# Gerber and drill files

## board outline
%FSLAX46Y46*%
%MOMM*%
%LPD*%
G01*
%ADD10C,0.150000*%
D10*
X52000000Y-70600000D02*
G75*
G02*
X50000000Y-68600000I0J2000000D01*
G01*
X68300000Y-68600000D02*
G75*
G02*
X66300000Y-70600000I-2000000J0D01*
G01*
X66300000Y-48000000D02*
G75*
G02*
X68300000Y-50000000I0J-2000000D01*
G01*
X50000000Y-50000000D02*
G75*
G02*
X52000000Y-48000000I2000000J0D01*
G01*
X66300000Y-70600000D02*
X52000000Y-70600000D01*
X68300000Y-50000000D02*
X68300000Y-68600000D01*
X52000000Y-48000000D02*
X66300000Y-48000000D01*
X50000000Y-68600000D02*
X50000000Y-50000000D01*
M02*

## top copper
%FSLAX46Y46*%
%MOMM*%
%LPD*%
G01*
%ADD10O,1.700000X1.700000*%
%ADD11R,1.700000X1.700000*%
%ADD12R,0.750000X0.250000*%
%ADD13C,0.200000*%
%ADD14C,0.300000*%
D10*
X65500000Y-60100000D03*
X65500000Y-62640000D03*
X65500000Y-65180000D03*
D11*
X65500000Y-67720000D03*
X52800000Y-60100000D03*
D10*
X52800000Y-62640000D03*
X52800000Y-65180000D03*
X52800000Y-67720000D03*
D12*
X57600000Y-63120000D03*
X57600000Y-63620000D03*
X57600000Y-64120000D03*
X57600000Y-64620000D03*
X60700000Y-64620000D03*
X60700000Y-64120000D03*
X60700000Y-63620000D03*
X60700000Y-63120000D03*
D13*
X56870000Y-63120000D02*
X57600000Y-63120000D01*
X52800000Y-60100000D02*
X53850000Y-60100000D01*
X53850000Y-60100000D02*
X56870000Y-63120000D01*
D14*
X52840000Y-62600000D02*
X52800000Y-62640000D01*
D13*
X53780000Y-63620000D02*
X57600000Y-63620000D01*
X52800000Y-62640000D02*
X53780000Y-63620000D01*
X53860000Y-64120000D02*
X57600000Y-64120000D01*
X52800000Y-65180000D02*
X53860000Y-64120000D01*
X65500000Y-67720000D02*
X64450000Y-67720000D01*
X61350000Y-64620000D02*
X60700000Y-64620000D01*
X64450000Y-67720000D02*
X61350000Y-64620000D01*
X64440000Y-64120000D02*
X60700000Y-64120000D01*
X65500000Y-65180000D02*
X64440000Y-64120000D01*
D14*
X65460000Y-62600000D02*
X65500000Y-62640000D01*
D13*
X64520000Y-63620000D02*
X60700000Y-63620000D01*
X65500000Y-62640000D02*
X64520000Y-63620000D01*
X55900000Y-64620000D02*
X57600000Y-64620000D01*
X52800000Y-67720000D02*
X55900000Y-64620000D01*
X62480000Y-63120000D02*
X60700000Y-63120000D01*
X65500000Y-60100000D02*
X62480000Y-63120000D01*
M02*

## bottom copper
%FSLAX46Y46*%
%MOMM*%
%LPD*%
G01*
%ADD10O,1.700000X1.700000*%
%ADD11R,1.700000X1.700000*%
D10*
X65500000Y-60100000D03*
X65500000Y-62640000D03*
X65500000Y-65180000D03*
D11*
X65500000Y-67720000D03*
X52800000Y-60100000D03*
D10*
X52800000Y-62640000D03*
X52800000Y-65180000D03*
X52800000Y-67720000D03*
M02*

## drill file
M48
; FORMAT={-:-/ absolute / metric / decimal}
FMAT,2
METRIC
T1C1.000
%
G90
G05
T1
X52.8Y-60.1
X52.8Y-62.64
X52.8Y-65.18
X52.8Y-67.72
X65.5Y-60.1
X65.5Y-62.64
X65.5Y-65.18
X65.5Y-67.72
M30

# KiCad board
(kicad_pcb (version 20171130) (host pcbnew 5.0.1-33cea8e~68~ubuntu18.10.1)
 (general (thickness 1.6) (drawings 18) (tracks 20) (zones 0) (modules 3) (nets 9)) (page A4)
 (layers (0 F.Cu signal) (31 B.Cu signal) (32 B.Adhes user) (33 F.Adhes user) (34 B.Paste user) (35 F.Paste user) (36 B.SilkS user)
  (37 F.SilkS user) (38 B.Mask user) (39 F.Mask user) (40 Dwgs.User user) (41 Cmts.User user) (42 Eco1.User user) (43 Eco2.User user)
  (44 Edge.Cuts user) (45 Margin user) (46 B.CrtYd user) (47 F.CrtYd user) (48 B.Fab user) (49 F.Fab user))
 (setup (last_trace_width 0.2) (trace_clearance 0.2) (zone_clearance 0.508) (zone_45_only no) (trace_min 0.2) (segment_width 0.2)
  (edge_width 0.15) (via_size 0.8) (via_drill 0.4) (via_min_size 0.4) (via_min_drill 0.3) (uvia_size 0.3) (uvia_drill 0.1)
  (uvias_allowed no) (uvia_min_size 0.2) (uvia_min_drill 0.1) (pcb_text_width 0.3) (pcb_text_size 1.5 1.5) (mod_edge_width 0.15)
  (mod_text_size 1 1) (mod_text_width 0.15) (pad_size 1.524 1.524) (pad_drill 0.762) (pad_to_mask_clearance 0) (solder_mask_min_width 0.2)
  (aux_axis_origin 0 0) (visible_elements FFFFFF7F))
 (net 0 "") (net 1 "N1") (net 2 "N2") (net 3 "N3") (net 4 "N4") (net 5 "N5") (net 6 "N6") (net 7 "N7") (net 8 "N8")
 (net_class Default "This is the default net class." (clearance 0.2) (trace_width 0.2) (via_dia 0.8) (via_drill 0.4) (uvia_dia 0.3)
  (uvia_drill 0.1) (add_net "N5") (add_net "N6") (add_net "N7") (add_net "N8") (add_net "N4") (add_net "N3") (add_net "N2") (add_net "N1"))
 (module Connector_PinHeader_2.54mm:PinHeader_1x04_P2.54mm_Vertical (layer F.Cu) (at 65.5 67.72 180)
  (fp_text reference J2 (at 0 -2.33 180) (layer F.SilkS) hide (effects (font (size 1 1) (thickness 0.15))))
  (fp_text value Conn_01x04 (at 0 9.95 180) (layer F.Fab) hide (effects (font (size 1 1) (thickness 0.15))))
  (pad 4 thru_hole oval (at 0 7.62 180) (size 1.7 1.7) (drill 1) (layers *.Cu *.Mask) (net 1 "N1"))
  (pad 3 thru_hole oval (at 0 5.08 180) (size 1.7 1.7) (drill 1) (layers *.Cu *.Mask) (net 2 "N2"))
  (pad 2 thru_hole oval (at 0 2.54 180) (size 1.7 1.7) (drill 1) (layers *.Cu *.Mask) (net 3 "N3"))
  (pad 1 thru_hole rect (at 0 0 180) (size 1.7 1.7) (drill 1) (layers *.Cu *.Mask) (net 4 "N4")))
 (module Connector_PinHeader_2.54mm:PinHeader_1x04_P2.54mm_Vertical (layer F.Cu) (at 52.8 60.1)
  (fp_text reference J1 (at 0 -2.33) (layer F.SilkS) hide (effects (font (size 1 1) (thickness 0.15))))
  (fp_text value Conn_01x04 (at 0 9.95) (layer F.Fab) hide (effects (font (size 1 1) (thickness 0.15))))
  (pad 1 thru_hole rect (at 0 0) (size 1.7 1.7) (drill 1) (layers *.Cu *.Mask) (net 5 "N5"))
  (pad 2 thru_hole oval (at 0 2.54) (size 1.7 1.7) (drill 1) (layers *.Cu *.Mask) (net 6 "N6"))
  (pad 3 thru_hole oval (at 0 5.08) (size 1.7 1.7) (drill 1) (layers *.Cu *.Mask) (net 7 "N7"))
  (pad 4 thru_hole oval (at 0 7.62) (size 1.7 1.7) (drill 1) (layers *.Cu *.Mask) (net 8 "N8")))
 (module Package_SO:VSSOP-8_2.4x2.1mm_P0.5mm (layer F.Cu) (at 59.15 63.87)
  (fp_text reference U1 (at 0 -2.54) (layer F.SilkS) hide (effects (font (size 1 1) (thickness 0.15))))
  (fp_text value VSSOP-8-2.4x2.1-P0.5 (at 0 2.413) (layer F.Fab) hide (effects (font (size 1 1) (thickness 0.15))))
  (pad 1 smd rect (at -1.55 -0.75) (size 0.75 0.25) (layers F.Cu F.Paste F.Mask) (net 5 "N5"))
  (pad 2 smd rect (at -1.55 -0.25) (size 0.75 0.25) (layers F.Cu F.Paste F.Mask) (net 6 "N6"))
  (pad 3 smd rect (at -1.55 0.25) (size 0.75 0.25) (layers F.Cu F.Paste F.Mask) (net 7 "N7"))
  (pad 4 smd rect (at -1.55 0.75) (size 0.75 0.25) (layers F.Cu F.Paste F.Mask) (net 8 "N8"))
  (pad 5 smd rect (at 1.55 0.75) (size 0.75 0.25) (layers F.Cu F.Paste F.Mask) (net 4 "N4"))
  (pad 6 smd rect (at 1.55 0.25) (size 0.75 0.25) (layers F.Cu F.Paste F.Mask) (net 3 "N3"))
  (pad 7 smd rect (at 1.55 -0.25) (size 0.75 0.25) (layers F.Cu F.Paste F.Mask) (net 2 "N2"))
  (pad 8 smd rect (at 1.55 -0.75) (size 0.75 0.25) (layers F.Cu F.Paste F.Mask) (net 1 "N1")))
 (gr_arc (start 52 68.6) (end 50 68.6) (angle -90) (layer Edge.Cuts) (width 0.15))
 (gr_arc (start 66.3 68.6) (end 66.3 70.6) (angle -90) (layer Edge.Cuts) (width 0.15))
 (gr_arc (start 66.3 50) (end 68.3 50) (angle -90) (layer Edge.Cuts) (width 0.15))
 (gr_arc (start 52 50) (end 52 48) (angle -90) (layer Edge.Cuts) (width 0.15))
 (gr_line (start 66.3 70.6) (end 52 70.6) (layer Edge.Cuts) (width 0.15))
 (gr_line (start 68.3 50) (end 68.3 68.6) (layer Edge.Cuts) (width 0.15))
 (gr_line (start 52 48) (end 66.3 48) (layer Edge.Cuts) (width 0.15))
 (gr_line (start 50 68.6) (end 50 50) (layer Edge.Cuts) (width 0.15))
 (segment (start 56.87 63.12) (end 57.6 63.12) (width 0.2) (layer F.Cu) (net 5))
 (segment (start 52.8 60.1) (end 53.85 60.1) (width 0.2) (layer F.Cu) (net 5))
 (segment (start 53.85 60.1) (end 56.87 63.12) (width 0.2) (layer F.Cu) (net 5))
 (segment (start 52.84 62.6) (end 52.8 62.64) (width 0.3) (layer F.Cu) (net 6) (status 30))
 (segment (start 53.78 63.62) (end 57.6 63.62) (width 0.2) (layer F.Cu) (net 6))
 (segment (start 52.8 62.64) (end 53.78 63.62) (width 0.2) (layer F.Cu) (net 6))
 (segment (start 53.86 64.12) (end 57.6 64.12) (width 0.2) (layer F.Cu) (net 7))
 (segment (start 52.8 65.18) (end 53.86 64.12) (width 0.2) (layer F.Cu) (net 7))
 (segment (start 65.5 67.72) (end 64.45 67.72) (width 0.2) (layer F.Cu) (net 4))
 (segment (start 61.35 64.62) (end 60.7 64.62) (width 0.2) (layer F.Cu) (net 4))
 (segment (start 64.45 67.72) (end 61.35 64.62) (width 0.2) (layer F.Cu) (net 4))
 (segment (start 64.44 64.12) (end 60.7 64.12) (width 0.2) (layer F.Cu) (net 3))
 (segment (start 65.5 65.18) (end 64.44 64.12) (width 0.2) (layer F.Cu) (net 3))
 (segment (start 65.46 62.6) (end 65.5 62.64) (width 0.3) (layer F.Cu) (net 2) (status 30))
 (segment (start 64.52 63.62) (end 60.7 63.62) (width 0.2) (layer F.Cu) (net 2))
 (segment (start 65.5 62.64) (end 64.52 63.62) (width 0.2) (layer F.Cu) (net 2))
 (segment (start 55.9 64.62) (end 57.6 64.62) (width 0.2) (layer F.Cu) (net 8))
 (segment (start 52.8 67.72) (end 55.9 64.62) (width 0.2) (layer F.Cu) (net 8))
 (segment (start 62.48 63.12) (end 60.7 63.12) (width 0.2) (layer F.Cu) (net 1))
 (segment (start 65.5 60.1) (end 62.48 63.12) (width 0.2) (layer F.Cu) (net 1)))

